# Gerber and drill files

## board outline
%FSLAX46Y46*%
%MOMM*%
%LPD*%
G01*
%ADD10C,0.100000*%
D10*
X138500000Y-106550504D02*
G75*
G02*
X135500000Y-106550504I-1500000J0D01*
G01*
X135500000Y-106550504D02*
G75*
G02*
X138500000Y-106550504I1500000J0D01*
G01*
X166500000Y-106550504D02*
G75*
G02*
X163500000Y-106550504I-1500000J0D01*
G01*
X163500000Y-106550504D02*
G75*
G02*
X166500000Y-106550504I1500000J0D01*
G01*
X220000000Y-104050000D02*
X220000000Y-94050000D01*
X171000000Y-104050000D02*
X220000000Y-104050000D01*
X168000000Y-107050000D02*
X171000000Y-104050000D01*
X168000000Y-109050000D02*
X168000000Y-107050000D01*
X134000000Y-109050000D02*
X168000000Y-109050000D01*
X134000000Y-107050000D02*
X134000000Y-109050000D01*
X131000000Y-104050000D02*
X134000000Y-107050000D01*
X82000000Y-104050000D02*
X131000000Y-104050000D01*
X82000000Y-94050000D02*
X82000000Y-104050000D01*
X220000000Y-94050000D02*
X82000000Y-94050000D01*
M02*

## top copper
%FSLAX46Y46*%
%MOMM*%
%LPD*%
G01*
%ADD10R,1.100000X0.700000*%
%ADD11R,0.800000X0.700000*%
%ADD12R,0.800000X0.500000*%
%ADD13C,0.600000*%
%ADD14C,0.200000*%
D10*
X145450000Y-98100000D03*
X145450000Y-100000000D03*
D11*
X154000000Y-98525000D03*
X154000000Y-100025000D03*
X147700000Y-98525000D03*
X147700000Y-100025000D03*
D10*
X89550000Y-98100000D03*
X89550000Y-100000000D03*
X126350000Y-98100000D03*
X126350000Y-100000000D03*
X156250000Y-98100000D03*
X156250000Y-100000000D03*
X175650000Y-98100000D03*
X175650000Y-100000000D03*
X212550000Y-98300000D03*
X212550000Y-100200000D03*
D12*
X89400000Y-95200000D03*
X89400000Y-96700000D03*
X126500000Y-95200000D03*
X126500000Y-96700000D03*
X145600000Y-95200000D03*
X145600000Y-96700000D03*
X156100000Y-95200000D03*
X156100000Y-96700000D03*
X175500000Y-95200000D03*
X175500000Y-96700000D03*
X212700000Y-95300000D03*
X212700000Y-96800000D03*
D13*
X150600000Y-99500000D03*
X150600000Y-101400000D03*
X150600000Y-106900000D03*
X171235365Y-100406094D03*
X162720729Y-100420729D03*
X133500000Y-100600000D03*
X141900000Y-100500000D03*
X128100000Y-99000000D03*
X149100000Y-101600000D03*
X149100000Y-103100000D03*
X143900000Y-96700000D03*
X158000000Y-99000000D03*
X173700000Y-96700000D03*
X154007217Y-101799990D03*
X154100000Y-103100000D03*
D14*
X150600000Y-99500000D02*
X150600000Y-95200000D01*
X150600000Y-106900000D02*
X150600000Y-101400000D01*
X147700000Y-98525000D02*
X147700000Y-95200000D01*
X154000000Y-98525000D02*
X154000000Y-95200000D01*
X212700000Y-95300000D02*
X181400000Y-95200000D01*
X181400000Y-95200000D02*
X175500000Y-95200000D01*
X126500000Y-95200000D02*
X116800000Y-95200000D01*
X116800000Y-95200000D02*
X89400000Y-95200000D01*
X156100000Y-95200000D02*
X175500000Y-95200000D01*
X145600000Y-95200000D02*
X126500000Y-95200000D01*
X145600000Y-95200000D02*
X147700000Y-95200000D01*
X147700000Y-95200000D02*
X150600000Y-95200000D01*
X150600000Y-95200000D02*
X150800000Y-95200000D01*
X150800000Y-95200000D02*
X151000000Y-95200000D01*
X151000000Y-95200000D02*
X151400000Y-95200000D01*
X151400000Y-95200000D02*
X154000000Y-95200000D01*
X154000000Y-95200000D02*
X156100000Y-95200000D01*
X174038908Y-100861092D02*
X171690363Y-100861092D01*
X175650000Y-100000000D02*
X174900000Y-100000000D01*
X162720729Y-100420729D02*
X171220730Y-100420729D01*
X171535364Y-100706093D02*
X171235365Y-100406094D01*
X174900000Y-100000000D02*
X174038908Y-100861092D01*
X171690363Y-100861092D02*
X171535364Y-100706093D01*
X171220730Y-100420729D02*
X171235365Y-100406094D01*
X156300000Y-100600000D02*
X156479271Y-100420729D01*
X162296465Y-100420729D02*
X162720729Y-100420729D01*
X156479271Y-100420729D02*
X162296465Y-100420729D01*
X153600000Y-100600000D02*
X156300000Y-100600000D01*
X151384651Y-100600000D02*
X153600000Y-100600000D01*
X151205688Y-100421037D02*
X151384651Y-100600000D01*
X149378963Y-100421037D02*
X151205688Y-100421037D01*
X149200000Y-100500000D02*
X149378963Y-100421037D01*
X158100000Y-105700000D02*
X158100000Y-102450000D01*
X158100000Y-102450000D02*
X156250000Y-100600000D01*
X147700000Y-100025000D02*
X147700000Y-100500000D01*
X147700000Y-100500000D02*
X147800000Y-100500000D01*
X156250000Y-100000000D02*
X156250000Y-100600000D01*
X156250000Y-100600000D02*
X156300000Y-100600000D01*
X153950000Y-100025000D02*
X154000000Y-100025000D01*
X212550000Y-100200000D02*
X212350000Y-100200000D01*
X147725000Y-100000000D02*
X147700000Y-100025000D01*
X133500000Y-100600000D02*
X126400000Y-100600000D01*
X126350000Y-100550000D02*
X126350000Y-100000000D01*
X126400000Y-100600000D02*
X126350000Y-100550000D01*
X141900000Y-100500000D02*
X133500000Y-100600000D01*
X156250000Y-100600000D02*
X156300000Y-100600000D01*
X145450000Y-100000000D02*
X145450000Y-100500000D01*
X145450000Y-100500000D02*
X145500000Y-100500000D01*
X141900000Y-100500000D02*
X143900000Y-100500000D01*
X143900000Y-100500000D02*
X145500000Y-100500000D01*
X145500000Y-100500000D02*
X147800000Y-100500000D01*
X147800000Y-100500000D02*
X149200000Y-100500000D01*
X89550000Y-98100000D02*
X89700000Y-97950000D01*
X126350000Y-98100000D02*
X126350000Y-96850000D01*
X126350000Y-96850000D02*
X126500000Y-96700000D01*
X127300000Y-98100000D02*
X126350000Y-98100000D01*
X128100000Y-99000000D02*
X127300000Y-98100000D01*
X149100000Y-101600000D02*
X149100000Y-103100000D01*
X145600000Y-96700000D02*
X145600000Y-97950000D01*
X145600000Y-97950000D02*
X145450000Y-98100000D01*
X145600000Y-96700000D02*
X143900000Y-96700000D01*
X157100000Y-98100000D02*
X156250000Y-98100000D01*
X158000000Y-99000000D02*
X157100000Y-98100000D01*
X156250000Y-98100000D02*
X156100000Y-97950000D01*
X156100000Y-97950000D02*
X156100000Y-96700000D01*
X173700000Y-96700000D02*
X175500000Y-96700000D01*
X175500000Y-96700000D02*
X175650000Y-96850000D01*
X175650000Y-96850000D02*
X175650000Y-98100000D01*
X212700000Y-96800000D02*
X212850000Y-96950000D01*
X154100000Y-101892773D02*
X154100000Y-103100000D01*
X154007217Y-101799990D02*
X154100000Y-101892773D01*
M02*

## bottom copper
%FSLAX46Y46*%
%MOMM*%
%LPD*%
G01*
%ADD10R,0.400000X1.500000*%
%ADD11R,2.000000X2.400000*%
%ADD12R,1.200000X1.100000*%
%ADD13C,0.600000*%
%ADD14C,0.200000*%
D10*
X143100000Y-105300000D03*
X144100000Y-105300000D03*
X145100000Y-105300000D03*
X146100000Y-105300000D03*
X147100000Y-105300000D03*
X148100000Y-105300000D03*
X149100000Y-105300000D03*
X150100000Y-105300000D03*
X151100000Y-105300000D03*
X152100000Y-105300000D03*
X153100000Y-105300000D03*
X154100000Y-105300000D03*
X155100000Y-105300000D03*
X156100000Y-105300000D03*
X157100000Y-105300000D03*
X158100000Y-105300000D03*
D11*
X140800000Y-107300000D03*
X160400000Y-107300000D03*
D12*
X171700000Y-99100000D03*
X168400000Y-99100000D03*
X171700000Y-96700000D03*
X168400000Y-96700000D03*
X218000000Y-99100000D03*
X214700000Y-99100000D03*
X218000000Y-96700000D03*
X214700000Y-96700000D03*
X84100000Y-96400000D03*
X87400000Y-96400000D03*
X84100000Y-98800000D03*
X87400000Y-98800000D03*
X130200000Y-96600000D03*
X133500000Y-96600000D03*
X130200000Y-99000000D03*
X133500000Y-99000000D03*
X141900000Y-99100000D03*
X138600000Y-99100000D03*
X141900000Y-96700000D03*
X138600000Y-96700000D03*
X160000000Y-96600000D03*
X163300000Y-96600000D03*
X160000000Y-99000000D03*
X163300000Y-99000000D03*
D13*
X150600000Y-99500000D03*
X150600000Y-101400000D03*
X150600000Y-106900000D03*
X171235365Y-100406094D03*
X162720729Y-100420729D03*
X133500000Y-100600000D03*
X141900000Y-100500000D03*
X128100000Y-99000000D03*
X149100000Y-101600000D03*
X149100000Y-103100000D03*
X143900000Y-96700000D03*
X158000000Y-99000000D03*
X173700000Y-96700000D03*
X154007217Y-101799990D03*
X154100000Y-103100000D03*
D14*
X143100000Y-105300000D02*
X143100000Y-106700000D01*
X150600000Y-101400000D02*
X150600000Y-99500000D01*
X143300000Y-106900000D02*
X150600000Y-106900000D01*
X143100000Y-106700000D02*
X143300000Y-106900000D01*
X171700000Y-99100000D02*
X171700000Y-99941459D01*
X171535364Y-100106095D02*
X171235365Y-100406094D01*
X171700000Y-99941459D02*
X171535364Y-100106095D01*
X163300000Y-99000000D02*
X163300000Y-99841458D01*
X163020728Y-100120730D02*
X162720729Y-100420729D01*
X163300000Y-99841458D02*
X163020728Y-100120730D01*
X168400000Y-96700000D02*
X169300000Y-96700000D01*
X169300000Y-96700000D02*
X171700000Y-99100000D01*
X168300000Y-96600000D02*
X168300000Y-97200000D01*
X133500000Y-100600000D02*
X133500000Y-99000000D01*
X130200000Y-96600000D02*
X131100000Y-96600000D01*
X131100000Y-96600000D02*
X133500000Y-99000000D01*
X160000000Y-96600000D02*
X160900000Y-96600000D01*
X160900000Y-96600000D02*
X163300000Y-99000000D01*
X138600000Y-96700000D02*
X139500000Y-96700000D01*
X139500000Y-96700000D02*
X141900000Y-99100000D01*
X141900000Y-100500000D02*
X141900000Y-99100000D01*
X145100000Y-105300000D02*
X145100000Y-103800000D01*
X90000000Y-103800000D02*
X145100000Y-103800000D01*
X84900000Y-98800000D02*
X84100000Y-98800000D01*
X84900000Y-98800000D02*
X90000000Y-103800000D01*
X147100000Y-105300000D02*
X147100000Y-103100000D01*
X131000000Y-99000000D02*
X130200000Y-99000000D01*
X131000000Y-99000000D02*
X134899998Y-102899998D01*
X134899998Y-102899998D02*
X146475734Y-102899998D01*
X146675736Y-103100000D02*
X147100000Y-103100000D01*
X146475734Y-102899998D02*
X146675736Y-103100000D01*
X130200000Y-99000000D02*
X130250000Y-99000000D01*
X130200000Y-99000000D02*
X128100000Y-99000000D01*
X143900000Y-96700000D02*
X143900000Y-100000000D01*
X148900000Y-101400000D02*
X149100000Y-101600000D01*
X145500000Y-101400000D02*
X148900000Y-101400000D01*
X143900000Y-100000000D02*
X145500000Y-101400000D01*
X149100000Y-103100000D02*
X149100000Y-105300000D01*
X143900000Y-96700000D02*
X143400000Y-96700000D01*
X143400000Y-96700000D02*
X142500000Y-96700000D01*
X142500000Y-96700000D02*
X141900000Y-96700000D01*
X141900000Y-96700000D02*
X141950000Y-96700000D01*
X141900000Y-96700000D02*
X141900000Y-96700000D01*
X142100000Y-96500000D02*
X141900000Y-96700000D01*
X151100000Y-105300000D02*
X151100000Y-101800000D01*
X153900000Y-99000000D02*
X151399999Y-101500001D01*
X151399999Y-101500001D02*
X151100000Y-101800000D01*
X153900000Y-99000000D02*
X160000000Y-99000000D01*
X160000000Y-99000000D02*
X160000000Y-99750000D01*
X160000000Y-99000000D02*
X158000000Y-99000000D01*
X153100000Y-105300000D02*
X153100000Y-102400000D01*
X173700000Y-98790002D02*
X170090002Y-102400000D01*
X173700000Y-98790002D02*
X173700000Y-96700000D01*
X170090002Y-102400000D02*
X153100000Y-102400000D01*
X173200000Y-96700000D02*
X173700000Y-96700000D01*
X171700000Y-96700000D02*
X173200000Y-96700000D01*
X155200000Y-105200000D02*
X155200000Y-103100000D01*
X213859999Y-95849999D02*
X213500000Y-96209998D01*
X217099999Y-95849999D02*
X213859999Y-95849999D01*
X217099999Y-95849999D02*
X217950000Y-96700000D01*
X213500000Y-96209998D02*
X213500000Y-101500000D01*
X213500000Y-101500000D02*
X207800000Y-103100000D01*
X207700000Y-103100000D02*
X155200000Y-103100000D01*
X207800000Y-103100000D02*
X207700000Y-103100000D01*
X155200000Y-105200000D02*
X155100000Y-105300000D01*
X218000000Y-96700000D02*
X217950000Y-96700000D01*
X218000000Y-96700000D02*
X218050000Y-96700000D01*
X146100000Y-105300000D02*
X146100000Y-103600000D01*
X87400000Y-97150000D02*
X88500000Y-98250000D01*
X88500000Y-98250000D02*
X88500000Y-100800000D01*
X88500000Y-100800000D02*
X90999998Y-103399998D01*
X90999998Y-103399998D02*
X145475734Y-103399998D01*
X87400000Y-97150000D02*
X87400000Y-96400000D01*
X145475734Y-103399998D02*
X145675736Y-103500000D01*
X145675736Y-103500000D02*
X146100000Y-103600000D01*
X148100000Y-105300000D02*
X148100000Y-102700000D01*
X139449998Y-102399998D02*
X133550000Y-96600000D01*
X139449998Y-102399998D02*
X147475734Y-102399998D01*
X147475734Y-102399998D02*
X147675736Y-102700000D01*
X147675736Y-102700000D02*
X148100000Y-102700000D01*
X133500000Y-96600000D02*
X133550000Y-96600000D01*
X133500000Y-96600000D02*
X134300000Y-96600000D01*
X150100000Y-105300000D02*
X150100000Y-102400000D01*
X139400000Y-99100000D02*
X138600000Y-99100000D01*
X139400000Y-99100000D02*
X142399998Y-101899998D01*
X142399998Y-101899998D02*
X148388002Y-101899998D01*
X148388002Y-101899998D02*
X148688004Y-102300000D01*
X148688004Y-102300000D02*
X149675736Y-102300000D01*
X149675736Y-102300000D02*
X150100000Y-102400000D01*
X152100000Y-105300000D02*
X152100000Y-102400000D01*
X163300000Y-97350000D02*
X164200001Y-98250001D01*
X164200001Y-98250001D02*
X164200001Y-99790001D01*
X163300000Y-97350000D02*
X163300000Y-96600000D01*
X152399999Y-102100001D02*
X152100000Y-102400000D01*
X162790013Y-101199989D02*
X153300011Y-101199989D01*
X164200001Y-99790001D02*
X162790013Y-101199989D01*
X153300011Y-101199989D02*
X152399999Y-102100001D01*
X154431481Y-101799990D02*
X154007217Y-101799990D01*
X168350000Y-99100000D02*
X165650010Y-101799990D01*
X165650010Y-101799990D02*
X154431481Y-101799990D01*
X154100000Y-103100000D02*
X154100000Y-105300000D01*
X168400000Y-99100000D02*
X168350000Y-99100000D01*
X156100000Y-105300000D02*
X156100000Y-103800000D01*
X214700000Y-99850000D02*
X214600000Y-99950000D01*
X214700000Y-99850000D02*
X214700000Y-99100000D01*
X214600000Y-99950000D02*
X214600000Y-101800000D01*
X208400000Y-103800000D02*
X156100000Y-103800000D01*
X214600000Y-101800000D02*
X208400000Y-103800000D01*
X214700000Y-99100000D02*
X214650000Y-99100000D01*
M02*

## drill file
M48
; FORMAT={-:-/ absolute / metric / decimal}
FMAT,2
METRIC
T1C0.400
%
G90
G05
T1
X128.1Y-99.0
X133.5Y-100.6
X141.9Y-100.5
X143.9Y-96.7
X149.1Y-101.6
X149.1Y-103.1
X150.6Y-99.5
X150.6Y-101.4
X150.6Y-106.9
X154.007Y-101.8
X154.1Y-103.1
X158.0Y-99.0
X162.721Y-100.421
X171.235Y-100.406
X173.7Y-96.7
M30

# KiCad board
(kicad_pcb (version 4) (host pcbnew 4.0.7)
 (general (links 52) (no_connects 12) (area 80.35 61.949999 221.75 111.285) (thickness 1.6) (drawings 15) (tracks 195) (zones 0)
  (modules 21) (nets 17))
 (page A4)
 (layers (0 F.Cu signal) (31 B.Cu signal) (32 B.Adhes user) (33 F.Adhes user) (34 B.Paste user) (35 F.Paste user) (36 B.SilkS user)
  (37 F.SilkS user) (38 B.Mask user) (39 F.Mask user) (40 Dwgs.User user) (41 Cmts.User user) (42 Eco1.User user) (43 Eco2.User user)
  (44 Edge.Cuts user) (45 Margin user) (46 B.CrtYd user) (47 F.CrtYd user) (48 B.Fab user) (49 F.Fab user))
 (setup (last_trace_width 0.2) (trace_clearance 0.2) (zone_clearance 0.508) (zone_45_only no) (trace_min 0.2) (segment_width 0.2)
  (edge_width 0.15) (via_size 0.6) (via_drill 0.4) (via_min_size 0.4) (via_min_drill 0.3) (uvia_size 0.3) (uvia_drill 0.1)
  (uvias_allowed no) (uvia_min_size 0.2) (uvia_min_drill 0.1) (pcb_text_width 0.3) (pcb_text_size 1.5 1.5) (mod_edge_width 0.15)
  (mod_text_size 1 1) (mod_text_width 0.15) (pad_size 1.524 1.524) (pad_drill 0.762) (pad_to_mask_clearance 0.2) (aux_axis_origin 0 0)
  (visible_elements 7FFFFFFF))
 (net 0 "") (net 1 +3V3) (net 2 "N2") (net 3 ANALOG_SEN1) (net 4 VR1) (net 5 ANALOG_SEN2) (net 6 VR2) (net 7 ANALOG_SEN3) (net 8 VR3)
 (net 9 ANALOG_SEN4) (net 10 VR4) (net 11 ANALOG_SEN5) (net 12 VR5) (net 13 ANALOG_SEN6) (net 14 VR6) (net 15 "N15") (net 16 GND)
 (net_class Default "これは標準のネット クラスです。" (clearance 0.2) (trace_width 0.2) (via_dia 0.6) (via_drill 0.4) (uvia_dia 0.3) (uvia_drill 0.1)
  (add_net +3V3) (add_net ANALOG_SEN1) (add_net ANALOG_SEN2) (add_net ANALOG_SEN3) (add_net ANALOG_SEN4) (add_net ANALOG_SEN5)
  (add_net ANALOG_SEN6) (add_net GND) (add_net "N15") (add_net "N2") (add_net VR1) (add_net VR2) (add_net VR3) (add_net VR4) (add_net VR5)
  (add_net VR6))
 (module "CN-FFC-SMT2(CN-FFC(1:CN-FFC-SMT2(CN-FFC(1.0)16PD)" (layer F.Cu) (at 140.1 110.3)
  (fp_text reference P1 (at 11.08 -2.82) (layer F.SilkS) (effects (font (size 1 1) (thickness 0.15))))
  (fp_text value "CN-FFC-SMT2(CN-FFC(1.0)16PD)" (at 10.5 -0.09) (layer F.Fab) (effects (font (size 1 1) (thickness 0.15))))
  (pad 1 smd rect (at 3 -5) (size 0.4 1.5) (layers B.Cu B.Paste B.Mask) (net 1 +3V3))
  (pad 2 smd rect (at 4 -5) (size 0.4 1.5) (layers B.Cu B.Paste B.Mask) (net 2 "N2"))
  (pad 3 smd rect (at 5 -5) (size 0.4 1.5) (layers B.Cu B.Paste B.Mask) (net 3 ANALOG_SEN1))
  (pad 4 smd rect (at 6 -5) (size 0.4 1.5) (layers B.Cu B.Paste B.Mask) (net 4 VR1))
  (pad 5 smd rect (at 7 -5) (size 0.4 1.5) (layers B.Cu B.Paste B.Mask) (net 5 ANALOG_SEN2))
  (pad 6 smd rect (at 8 -5) (size 0.4 1.5) (layers B.Cu B.Paste B.Mask) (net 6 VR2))
  (pad 7 smd rect (at 9 -5) (size 0.4 1.5) (layers B.Cu B.Paste B.Mask) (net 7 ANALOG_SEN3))
  (pad 8 smd rect (at 10 -5) (size 0.4 1.5) (layers B.Cu B.Paste B.Mask) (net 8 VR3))
  (pad 9 smd rect (at 11 -5) (size 0.4 1.5) (layers B.Cu B.Paste B.Mask) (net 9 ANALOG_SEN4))
  (pad 10 smd rect (at 12 -5) (size 0.4 1.5) (layers B.Cu B.Paste B.Mask) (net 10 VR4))
  (pad 11 smd rect (at 13 -5) (size 0.4 1.5) (layers B.Cu B.Paste B.Mask) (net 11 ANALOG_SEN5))
  (pad 12 smd rect (at 14 -5) (size 0.4 1.5) (layers B.Cu B.Paste B.Mask) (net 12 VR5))
  (pad 13 smd rect (at 15 -5) (size 0.4 1.5) (layers B.Cu B.Paste B.Mask) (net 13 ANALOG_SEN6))
  (pad 14 smd rect (at 16 -5) (size 0.4 1.5) (layers B.Cu B.Paste B.Mask) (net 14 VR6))
  (pad 15 smd rect (at 17 -5) (size 0.4 1.5) (layers B.Cu B.Paste B.Mask) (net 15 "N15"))
  (pad 16 smd rect (at 18 -5) (size 0.4 1.5) (layers B.Cu B.Paste B.Mask) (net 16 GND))
  (pad "" smd rect (at 0.7 -3) (size 2 2.4) (layers B.Cu B.Paste B.Mask))
  (pad "" smd rect (at 20.3 -3) (size 2 2.4) (layers B.Cu B.Paste B.Mask)))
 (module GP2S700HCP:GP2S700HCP (layer F.Cu) (at 175 93.1 180)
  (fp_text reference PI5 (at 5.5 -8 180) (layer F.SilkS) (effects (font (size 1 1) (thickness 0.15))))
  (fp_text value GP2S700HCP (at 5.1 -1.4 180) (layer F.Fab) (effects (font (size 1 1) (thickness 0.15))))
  (pad 1 smd rect (at 3.3 -6 180) (size 1.2 1.1) (layers B.Cu B.Paste B.Mask) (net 16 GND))
  (pad 4 smd rect (at 6.6 -6 180) (size 1.2 1.1) (layers B.Cu B.Paste B.Mask) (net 12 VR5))
  (pad 2 smd rect (at 3.3 -3.6 180) (size 1.2 1.1) (layers B.Cu B.Paste B.Mask) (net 11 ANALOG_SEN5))
  (pad 3 smd rect (at 6.6 -3.6 180) (size 1.2 1.1) (layers B.Cu B.Paste B.Mask) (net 16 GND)))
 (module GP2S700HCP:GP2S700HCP (layer F.Cu) (at 221.3 93.1 180)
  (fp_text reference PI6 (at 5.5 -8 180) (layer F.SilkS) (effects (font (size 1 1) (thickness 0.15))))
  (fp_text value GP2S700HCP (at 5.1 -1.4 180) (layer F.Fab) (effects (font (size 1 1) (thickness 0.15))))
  (pad 1 smd rect (at 3.3 -6 180) (size 1.2 1.1) (layers B.Cu B.Paste B.Mask) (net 16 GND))
  (pad 4 smd rect (at 6.6 -6 180) (size 1.2 1.1) (layers B.Cu B.Paste B.Mask) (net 14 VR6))
  (pad 2 smd rect (at 3.3 -3.6 180) (size 1.2 1.1) (layers B.Cu B.Paste B.Mask) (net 13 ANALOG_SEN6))
  (pad 3 smd rect (at 6.6 -3.6 180) (size 1.2 1.1) (layers B.Cu B.Paste B.Mask) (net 16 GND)))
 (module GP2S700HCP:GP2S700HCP (layer F.Cu) (at 80.8 102.4)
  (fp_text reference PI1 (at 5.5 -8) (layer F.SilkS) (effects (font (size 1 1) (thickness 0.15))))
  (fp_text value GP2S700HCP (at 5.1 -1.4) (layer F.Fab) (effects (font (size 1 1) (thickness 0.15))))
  (pad 1 smd rect (at 3.3 -6) (size 1.2 1.1) (layers B.Cu B.Paste B.Mask) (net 16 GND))
  (pad 4 smd rect (at 6.6 -6) (size 1.2 1.1) (layers B.Cu B.Paste B.Mask) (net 4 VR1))
  (pad 2 smd rect (at 3.3 -3.6) (size 1.2 1.1) (layers B.Cu B.Paste B.Mask) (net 3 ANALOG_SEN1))
  (pad 3 smd rect (at 6.6 -3.6) (size 1.2 1.1) (layers B.Cu B.Paste B.Mask) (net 16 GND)))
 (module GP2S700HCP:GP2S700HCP (layer F.Cu) (at 126.9 102.6)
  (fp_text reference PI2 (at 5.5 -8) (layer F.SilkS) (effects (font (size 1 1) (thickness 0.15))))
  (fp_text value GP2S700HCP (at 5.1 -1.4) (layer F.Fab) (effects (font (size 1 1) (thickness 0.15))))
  (pad 1 smd rect (at 3.3 -6) (size 1.2 1.1) (layers B.Cu B.Paste B.Mask) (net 16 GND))
  (pad 4 smd rect (at 6.6 -6) (size 1.2 1.1) (layers B.Cu B.Paste B.Mask) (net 6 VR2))
  (pad 2 smd rect (at 3.3 -3.6) (size 1.2 1.1) (layers B.Cu B.Paste B.Mask) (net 5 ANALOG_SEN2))
  (pad 3 smd rect (at 6.6 -3.6) (size 1.2 1.1) (layers B.Cu B.Paste B.Mask) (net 16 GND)))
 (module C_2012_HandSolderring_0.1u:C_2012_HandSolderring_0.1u (layer F.Cu) (at 143.5 96.7 270)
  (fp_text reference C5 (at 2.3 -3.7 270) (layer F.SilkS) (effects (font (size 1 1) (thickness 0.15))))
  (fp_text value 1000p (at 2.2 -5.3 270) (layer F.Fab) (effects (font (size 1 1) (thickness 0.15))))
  (pad 1 smd rect (at 1.4 -1.95 270) (size 0.7 1.1) (layers F.Cu F.Paste F.Mask) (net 7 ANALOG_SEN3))
  (pad 2 smd rect (at 3.3 -1.95 270) (size 0.7 1.1) (layers F.Cu F.Paste F.Mask) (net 16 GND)))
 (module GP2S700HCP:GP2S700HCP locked (layer F.Cu) (at 145.2 93.1 180)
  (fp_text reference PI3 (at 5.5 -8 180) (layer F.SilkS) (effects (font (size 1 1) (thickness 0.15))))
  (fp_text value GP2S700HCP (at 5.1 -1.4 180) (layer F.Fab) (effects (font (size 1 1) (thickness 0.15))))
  (pad 1 smd rect (at 3.3 -6 180) (size 1.2 1.1) (layers B.Cu B.Paste B.Mask) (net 16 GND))
  (pad 4 smd rect (at 6.6 -6 180) (size 1.2 1.1) (layers B.Cu B.Paste B.Mask) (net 8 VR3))
  (pad 2 smd rect (at 3.3 -3.6 180) (size 1.2 1.1) (layers B.Cu B.Paste B.Mask) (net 7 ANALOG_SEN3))
  (pad 3 smd rect (at 6.6 -3.6 180) (size 1.2 1.1) (layers B.Cu B.Paste B.Mask) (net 16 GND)))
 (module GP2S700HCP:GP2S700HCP (layer F.Cu) (at 156.7 102.6)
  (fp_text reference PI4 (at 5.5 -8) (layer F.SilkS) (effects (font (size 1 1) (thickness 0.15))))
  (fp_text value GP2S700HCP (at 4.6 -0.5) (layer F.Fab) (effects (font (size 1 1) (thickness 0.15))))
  (pad 1 smd rect (at 3.3 -6) (size 1.2 1.1) (layers B.Cu B.Paste B.Mask) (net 16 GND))
  (pad 4 smd rect (at 6.6 -6) (size 1.2 1.1) (layers B.Cu B.Paste B.Mask) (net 10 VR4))
  (pad 2 smd rect (at 3.3 -3.6) (size 1.2 1.1) (layers B.Cu B.Paste B.Mask) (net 9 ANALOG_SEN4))
  (pad 3 smd rect (at 6.6 -3.6) (size 1.2 1.1) (layers B.Cu B.Paste B.Mask) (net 16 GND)))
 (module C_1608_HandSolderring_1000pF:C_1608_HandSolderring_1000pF (layer F.Cu) (at 153.1 97.9 270)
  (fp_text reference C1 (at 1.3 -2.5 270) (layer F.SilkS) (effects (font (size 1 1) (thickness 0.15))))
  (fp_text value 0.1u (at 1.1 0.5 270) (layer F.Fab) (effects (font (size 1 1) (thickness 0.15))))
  (pad 1 smd rect (at 0.625 -0.9 270) (size 0.7 0.8) (layers F.Cu F.Paste F.Mask) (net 1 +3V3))
  (pad 2 smd rect (at 2.125 -0.9 270) (size 0.7 0.8) (layers F.Cu F.Paste F.Mask) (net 16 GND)))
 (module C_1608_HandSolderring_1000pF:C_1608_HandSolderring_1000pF (layer F.Cu) (at 146.8 97.9 270)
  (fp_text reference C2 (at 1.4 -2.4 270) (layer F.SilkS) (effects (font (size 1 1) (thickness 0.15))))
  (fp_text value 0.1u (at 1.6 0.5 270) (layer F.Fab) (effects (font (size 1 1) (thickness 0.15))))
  (pad 1 smd rect (at 0.625 -0.9 270) (size 0.7 0.8) (layers F.Cu F.Paste F.Mask) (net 1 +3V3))
  (pad 2 smd rect (at 2.125 -0.9 270) (size 0.7 0.8) (layers F.Cu F.Paste F.Mask) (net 16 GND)))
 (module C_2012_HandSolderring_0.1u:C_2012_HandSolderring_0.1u (layer F.Cu) (at 87.6 96.7 270)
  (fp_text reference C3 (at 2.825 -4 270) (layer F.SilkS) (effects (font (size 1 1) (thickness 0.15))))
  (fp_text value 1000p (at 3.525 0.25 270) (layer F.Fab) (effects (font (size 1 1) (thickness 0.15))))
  (pad 1 smd rect (at 1.4 -1.95 270) (size 0.7 1.1) (layers F.Cu F.Paste F.Mask) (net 3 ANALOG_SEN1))
  (pad 2 smd rect (at 3.3 -1.95 270) (size 0.7 1.1) (layers F.Cu F.Paste F.Mask) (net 16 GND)))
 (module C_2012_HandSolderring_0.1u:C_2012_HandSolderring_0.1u (layer F.Cu) (at 124.4 96.7 270)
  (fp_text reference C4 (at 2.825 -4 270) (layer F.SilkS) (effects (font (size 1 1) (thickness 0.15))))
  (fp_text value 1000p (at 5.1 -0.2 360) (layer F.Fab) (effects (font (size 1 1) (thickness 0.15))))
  (pad 1 smd rect (at 1.4 -1.95 270) (size 0.7 1.1) (layers F.Cu F.Paste F.Mask) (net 5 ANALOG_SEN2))
  (pad 2 smd rect (at 3.3 -1.95 270) (size 0.7 1.1) (layers F.Cu F.Paste F.Mask) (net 16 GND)))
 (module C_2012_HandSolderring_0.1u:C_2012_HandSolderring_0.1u (layer F.Cu) (at 154.3 96.7 270)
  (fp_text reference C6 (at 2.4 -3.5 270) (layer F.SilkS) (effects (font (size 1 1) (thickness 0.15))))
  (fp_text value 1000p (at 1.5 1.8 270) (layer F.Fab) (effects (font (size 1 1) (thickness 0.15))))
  (pad 1 smd rect (at 1.4 -1.95 270) (size 0.7 1.1) (layers F.Cu F.Paste F.Mask) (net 9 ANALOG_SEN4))
  (pad 2 smd rect (at 3.3 -1.95 270) (size 0.7 1.1) (layers F.Cu F.Paste F.Mask) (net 16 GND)))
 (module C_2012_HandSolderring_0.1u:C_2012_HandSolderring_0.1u (layer F.Cu) (at 173.7 96.7 270)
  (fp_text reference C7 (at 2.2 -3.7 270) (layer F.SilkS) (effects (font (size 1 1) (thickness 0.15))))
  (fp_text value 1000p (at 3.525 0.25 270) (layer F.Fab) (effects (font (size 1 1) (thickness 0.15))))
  (pad 1 smd rect (at 1.4 -1.95 270) (size 0.7 1.1) (layers F.Cu F.Paste F.Mask) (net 11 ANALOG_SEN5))
  (pad 2 smd rect (at 3.3 -1.95 270) (size 0.7 1.1) (layers F.Cu F.Paste F.Mask) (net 16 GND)))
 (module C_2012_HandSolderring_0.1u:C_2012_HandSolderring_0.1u (layer F.Cu) (at 210.6 96.9 270)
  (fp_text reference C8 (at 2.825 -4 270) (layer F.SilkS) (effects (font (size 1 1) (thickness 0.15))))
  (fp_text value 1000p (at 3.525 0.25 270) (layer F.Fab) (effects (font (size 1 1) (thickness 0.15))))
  (pad 1 smd rect (at 1.4 -1.95 270) (size 0.7 1.1) (layers F.Cu F.Paste F.Mask) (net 13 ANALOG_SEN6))
  (pad 2 smd rect (at 3.3 -1.95 270) (size 0.7 1.1) (layers F.Cu F.Paste F.Mask) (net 16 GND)))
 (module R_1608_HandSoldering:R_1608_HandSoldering (layer F.Cu) (at 87.8 93.8 270)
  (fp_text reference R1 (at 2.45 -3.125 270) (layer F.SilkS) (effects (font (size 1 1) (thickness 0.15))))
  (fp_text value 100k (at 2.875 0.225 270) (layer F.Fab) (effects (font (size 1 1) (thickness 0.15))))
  (pad 1 smd rect (at 1.4 -1.6 270) (size 0.5 0.8) (layers F.Cu F.Paste F.Mask) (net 1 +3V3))
  (pad 2 smd rect (at 2.9 -1.6 270) (size 0.5 0.8) (layers F.Cu F.Paste F.Mask) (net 3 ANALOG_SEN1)))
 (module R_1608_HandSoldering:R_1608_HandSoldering (layer F.Cu) (at 124.9 93.8 270)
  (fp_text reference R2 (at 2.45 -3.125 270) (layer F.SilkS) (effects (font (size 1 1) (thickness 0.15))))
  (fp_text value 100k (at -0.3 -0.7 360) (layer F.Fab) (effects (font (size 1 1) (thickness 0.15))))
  (pad 1 smd rect (at 1.4 -1.6 270) (size 0.5 0.8) (layers F.Cu F.Paste F.Mask) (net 1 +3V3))
  (pad 2 smd rect (at 2.9 -1.6 270) (size 0.5 0.8) (layers F.Cu F.Paste F.Mask) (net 5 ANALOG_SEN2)))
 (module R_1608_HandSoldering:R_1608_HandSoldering (layer F.Cu) (at 144 93.8 270)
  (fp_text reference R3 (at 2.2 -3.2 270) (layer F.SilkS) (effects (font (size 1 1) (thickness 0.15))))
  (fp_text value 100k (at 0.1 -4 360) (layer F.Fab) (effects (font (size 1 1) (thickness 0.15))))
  (pad 1 smd rect (at 1.4 -1.6 270) (size 0.5 0.8) (layers F.Cu F.Paste F.Mask) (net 1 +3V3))
  (pad 2 smd rect (at 2.9 -1.6 270) (size 0.5 0.8) (layers F.Cu F.Paste F.Mask) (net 7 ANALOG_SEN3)))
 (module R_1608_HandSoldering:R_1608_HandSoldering (layer F.Cu) (at 154.5 93.8 270)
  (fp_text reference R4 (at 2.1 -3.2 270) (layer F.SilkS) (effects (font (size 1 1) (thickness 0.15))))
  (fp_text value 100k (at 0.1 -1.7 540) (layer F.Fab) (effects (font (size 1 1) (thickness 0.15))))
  (pad 1 smd rect (at 1.4 -1.6 270) (size 0.5 0.8) (layers F.Cu F.Paste F.Mask) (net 1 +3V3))
  (pad 2 smd rect (at 2.9 -1.6 270) (size 0.5 0.8) (layers F.Cu F.Paste F.Mask) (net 9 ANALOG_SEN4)))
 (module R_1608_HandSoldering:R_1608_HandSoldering (layer F.Cu) (at 173.9 93.8 270)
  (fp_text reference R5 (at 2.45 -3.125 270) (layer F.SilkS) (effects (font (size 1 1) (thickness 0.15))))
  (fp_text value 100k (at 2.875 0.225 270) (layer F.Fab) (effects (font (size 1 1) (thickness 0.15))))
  (pad 1 smd rect (at 1.4 -1.6 270) (size 0.5 0.8) (layers F.Cu F.Paste F.Mask) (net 1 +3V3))
  (pad 2 smd rect (at 2.9 -1.6 270) (size 0.5 0.8) (layers F.Cu F.Paste F.Mask) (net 11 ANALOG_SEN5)))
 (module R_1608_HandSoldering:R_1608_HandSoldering (layer F.Cu) (at 211.1 93.9 270)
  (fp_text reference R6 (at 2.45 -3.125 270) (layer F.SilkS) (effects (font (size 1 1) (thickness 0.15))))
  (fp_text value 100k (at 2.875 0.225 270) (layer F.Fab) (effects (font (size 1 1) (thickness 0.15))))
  (pad 1 smd rect (at 1.4 -1.6 270) (size 0.5 0.8) (layers F.Cu F.Paste F.Mask) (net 1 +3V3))
  (pad 2 smd rect (at 2.9 -1.6 270) (size 0.5 0.8) (layers F.Cu F.Paste F.Mask) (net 13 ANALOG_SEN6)))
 (gr_circle (center 137 106.550504) (end 137 105.050504) (layer Edge.Cuts) (width 0.1))
 (gr_circle (center 165 106.550504) (end 165 105.050504) (layer Edge.Cuts) (width 0.1))
 (gr_line (start 220 104.05) (end 220 94.05) (layer Edge.Cuts) (width 0.1))
 (gr_line (start 171 104.05) (end 220 104.05) (layer Edge.Cuts) (width 0.1))
 (gr_line (start 168 107.05) (end 171 104.05) (layer Edge.Cuts) (width 0.1))
 (gr_line (start 168 109.05) (end 168 107.05) (layer Edge.Cuts) (width 0.1))
 (gr_line (start 134 109.05) (end 168 109.05) (layer Edge.Cuts) (width 0.1))
 (gr_line (start 134 107.05) (end 134 109.05) (layer Edge.Cuts) (width 0.1))
 (gr_line (start 131 104.05) (end 134 107.05) (layer Edge.Cuts) (width 0.1))
 (gr_line (start 82 104.05) (end 131 104.05) (layer Edge.Cuts) (width 0.1))
 (gr_line (start 82 94.05) (end 82 104.05) (layer Edge.Cuts) (width 0.1))
 (gr_line (start 220 94.05) (end 82 94.05) (layer Edge.Cuts) (width 0.1))
 (segment (start 143.1 105.3) (end 143.1 106.7) (width 0.2) (layer B.Cu) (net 1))
 (segment (start 150.6 99.5) (end 150.6 95.2) (width 0.2) (layer F.Cu) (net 1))
 (via (at 150.6 99.5) (size 0.6) (drill 0.4) (layers F.Cu B.Cu) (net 1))
 (segment (start 150.6 101.4) (end 150.6 99.5) (width 0.2) (layer B.Cu) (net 1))
 (via (at 150.6 101.4) (size 0.6) (drill 0.4) (layers F.Cu B.Cu) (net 1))
 (segment (start 150.6 106.9) (end 150.6 101.4) (width 0.2) (layer F.Cu) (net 1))
 (via (at 150.6 106.9) (size 0.6) (drill 0.4) (layers F.Cu B.Cu) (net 1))
 (segment (start 143.3 106.9) (end 150.6 106.9) (width 0.2) (layer B.Cu) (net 1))
 (segment (start 143.1 106.7) (end 143.3 106.9) (width 0.2) (layer B.Cu) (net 1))
 (segment (start 147.7 98.525) (end 147.7 95.2) (width 0.2) (layer F.Cu) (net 1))
 (segment (start 154 98.525) (end 154 95.2) (width 0.2) (layer F.Cu) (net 1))
 (segment (start 212.7 95.3) (end 181.4 95.2) (width 0.2) (layer F.Cu) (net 1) (status 10))
 (segment (start 181.4 95.2) (end 175.5 95.2) (width 0.2) (layer F.Cu) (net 1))
 (segment (start 126.5 95.2) (end 116.8 95.2) (width 0.2) (layer F.Cu) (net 1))
 (segment (start 116.8 95.2) (end 89.4 95.2) (width 0.2) (layer F.Cu) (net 1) (status 20))
 (segment (start 156.1 95.2) (end 175.5 95.2) (width 0.2) (layer F.Cu) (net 1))
 (segment (start 145.6 95.2) (end 126.5 95.2) (width 0.2) (layer F.Cu) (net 1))
 (segment (start 145.6 95.2) (end 147.7 95.2) (width 0.2) (layer F.Cu) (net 1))
 (segment (start 147.7 95.2) (end 150.6 95.2) (width 0.2) (layer F.Cu) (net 1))
 (segment (start 150.6 95.2) (end 150.8 95.2) (width 0.2) (layer F.Cu) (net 1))
 (segment (start 150.8 95.2) (end 151 95.2) (width 0.2) (layer F.Cu) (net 1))
 (segment (start 151 95.2) (end 151.4 95.2) (width 0.2) (layer F.Cu) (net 1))
 (segment (start 151.4 95.2) (end 154 95.2) (width 0.2) (layer F.Cu) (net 1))
 (segment (start 154 95.2) (end 156.1 95.2) (width 0.2) (layer F.Cu) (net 1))
 (segment (start 174.038908 100.861092) (end 171.690363 100.861092) (width 0.2) (layer F.Cu) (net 16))
 (segment (start 175.65 100) (end 174.9 100) (width 0.2) (layer F.Cu) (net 16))
 (segment (start 171.7 99.1) (end 171.7 99.941459) (width 0.2) (layer B.Cu) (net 16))
 (segment (start 162.720729 100.420729) (end 171.22073 100.420729) (width 0.2) (layer F.Cu) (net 16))
 (segment (start 171.535364 100.706093) (end 171.235365 100.406094) (width 0.2) (layer F.Cu) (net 16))
 (segment (start 174.9 100) (end 174.038908 100.861092) (width 0.2) (layer F.Cu) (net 16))
 (segment (start 171.535364 100.106095) (end 171.235365 100.406094) (width 0.2) (layer B.Cu) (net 16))
 (segment (start 171.690363 100.861092) (end 171.535364 100.706093) (width 0.2) (layer F.Cu) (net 16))
 (segment (start 171.22073 100.420729) (end 171.235365 100.406094) (width 0.2) (layer F.Cu) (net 16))
 (via (at 171.235365 100.406094) (size 0.6) (drill 0.4) (layers F.Cu B.Cu) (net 16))
 (segment (start 171.7 99.941459) (end 171.535364 100.106095) (width 0.2) (layer B.Cu) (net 16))
 (segment (start 156.3 100.6) (end 156.479271 100.420729) (width 0.2) (layer F.Cu) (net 16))
 (segment (start 163.3 99) (end 163.3 99.841458) (width 0.2) (layer B.Cu) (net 16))
 (segment (start 163.020728 100.12073) (end 162.720729 100.420729) (width 0.2) (layer B.Cu) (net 16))
 (via (at 162.720729 100.420729) (size 0.6) (drill 0.4) (layers F.Cu B.Cu) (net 16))
 (segment (start 162.296465 100.420729) (end 162.720729 100.420729) (width 0.2) (layer F.Cu) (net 16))
 (segment (start 156.479271 100.420729) (end 162.296465 100.420729) (width 0.2) (layer F.Cu) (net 16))
 (segment (start 163.3 99.841458) (end 163.020728 100.12073) (width 0.2) (layer B.Cu) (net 16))
 (segment (start 153.6 100.6) (end 156.3 100.6) (width 0.2) (layer F.Cu) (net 16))
 (segment (start 151.384651 100.6) (end 153.6 100.6) (width 0.2) (layer F.Cu) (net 16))
 (segment (start 151.205688 100.421037) (end 151.384651 100.6) (width 0.2) (layer F.Cu) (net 16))
 (segment (start 149.378963 100.421037) (end 151.205688 100.421037) (width 0.2) (layer F.Cu) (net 16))
 (segment (start 149.2 100.5) (end 149.378963 100.421037) (width 0.2) (layer F.Cu) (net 16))
 (segment (start 158.1 105.7) (end 158.1 102.45) (width 0.2) (layer F.Cu) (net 16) (status 10))
 (segment (start 158.1 102.45) (end 156.25 100.6) (width 0.2) (layer F.Cu) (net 16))
 (segment (start 147.7 100.025) (end 147.7 100.5) (width 0.2) (layer F.Cu) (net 16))
 (segment (start 147.7 100.5) (end 147.8 100.5) (width 0.2) (layer F.Cu) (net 16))
 (segment (start 156.25 100) (end 156.25 100.6) (width 0.2) (layer F.Cu) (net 16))
 (segment (start 156.25 100.6) (end 156.3 100.6) (width 0.2) (layer F.Cu) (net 16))
 (segment (start 168.4 96.7) (end 169.3 96.7) (width 0.2) (layer B.Cu) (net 16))
 (segment (start 169.3 96.7) (end 171.7 99.1) (width 0.2) (layer B.Cu) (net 16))
 (segment (start 153.95 100.025) (end 154 100.025) (width 0.2) (layer F.Cu) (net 16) (status 30))
 (segment (start 212.55 100.2) (end 212.35 100.2) (width 0.2) (layer F.Cu) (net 16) (status 30))
 (segment (start 168.3 96.6) (end 168.3 97.2) (width 0.2) (layer B.Cu) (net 16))
 (segment (start 147.725 100) (end 147.7 100.025) (width 0.2) (layer F.Cu) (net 16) (status 30))
 (segment (start 133.5 100.6) (end 126.4 100.6) (width 0.2) (layer F.Cu) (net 16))
 (segment (start 126.35 100.55) (end 126.35 100) (width 0.2) (layer F.Cu) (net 16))
 (segment (start 126.4 100.6) (end 126.35 100.55) (width 0.2) (layer F.Cu) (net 16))
 (segment (start 141.9 100.5) (end 133.5 100.6) (width 0.2) (layer F.Cu) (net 16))
 (segment (start 133.5 100.6) (end 133.5 99) (width 0.2) (layer B.Cu) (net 16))
 (via (at 133.5 100.6) (size 0.6) (drill 0.4) (layers F.Cu B.Cu) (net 16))
 (segment (start 130.2 96.6) (end 131.1 96.6) (width 0.2) (layer B.Cu) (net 16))
 (segment (start 131.1 96.6) (end 133.5 99) (width 0.2) (layer B.Cu) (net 16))
 (segment (start 156.25 100.6) (end 156.3 100.6) (width 0.2) (layer F.Cu) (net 16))
 (segment (start 145.45 100) (end 145.45 100.5) (width 0.2) (layer F.Cu) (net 16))
 (segment (start 145.45 100.5) (end 145.5 100.5) (width 0.2) (layer F.Cu) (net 16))
 (segment (start 160 96.6) (end 160.9 96.6) (width 0.2) (layer B.Cu) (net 16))
 (segment (start 160.9 96.6) (end 163.3 99) (width 0.2) (layer B.Cu) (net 16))
 (segment (start 138.6 96.7) (end 139.5 96.7) (width 0.2) (layer B.Cu) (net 16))
 (segment (start 139.5 96.7) (end 141.9 99.1) (width 0.2) (layer B.Cu) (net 16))
 (segment (start 141.9 100.5) (end 143.9 100.5) (width 0.2) (layer F.Cu) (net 16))
 (segment (start 143.9 100.5) (end 145.5 100.5) (width 0.2) (layer F.Cu) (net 16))
 (segment (start 145.5 100.5) (end 147.8 100.5) (width 0.2) (layer F.Cu) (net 16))
 (segment (start 147.8 100.5) (end 149.2 100.5) (width 0.2) (layer F.Cu) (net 16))
 (segment (start 141.9 100.5) (end 141.9 99.1) (width 0.2) (layer B.Cu) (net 16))
 (via (at 141.9 100.5) (size 0.6) (drill 0.4) (layers F.Cu B.Cu) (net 16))
 (segment (start 145.1 105.3) (end 145.1 103.8) (width 0.2) (layer B.Cu) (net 3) (status 10))
 (segment (start 90 103.8) (end 145.1 103.8) (width 0.2) (layer B.Cu) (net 3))
 (segment (start 84.9 98.8) (end 84.1 98.8) (width 0.2) (layer B.Cu) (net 3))
 (segment (start 84.9 98.8) (end 90 103.8) (width 0.2) (layer B.Cu) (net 3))
 (segment (start 89.55 98.1) (end 89.7 97.95) (width 0.2) (layer F.Cu) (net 3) (status 30))
 (segment (start 147.1 105.3) (end 147.1 103.1) (width 0.2) (layer B.Cu) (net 5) (status 10))
 (segment (start 131 99) (end 130.2 99) (width 0.2) (layer B.Cu) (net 5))
 (segment (start 131 99) (end 134.899998 102.899998) (width 0.2) (layer B.Cu) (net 5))
 (segment (start 134.899998 102.899998) (end 146.475734 102.899998) (width 0.2) (layer B.Cu) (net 5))
 (segment (start 146.675736 103.1) (end 147.1 103.1) (width 0.2) (layer B.Cu) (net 5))
 (segment (start 146.475734 102.899998) (end 146.675736 103.1) (width 0.2) (layer B.Cu) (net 5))
 (segment (start 130.2 99) (end 130.25 99) (width 0.2) (layer B.Cu) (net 5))
 (segment (start 130.2 99) (end 128.1 99) (width 0.2) (layer B.Cu) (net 5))
 (via (at 128.1 99) (size 0.6) (drill 0.4) (layers F.Cu B.Cu) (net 5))
 (segment (start 126.35 98.1) (end 126.35 96.85) (width 0.2) (layer F.Cu) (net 5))
 (segment (start 126.35 96.85) (end 126.5 96.7) (width 0.2) (layer F.Cu) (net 5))
 (segment (start 127.3 98.1) (end 126.35 98.1) (width 0.2) (layer F.Cu) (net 5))
 (segment (start 128.1 99) (end 127.3 98.1) (width 0.2) (layer F.Cu) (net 5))
 (via (at 149.1 101.6) (size 0.6) (drill 0.4) (layers F.Cu B.Cu) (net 7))
 (segment (start 143.9 96.7) (end 143.9 100) (width 0.2) (layer B.Cu) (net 7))
 (segment (start 148.9 101.4) (end 149.1 101.6) (width 0.2) (layer B.Cu) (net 7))
 (segment (start 145.5 101.4) (end 148.9 101.4) (width 0.2) (layer B.Cu) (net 7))
 (segment (start 143.9 100) (end 145.5 101.4) (width 0.2) (layer B.Cu) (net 7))
 (segment (start 149.1 103.1) (end 149.1 105.3) (width 0.2) (layer B.Cu) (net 7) (status 20))
 (via (at 149.1 103.1) (size 0.6) (drill 0.4) (layers F.Cu B.Cu) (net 7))
 (segment (start 149.1 101.6) (end 149.1 103.1) (width 0.2) (layer F.Cu) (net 7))
 (segment (start 143.9 96.7) (end 143.4 96.7) (width 0.2) (layer B.Cu) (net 7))
 (segment (start 143.4 96.7) (end 142.5 96.7) (width 0.2) (layer B.Cu) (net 7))
 (segment (start 142.5 96.7) (end 141.9 96.7) (width 0.2) (layer B.Cu) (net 7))
 (segment (start 141.9 96.7) (end 141.95 96.7) (width 0.2) (layer B.Cu) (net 7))
 (segment (start 141.9 96.7) (end 141.9 96.7) (width 0.2) (layer B.Cu) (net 7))
 (segment (start 145.6 96.7) (end 145.6 97.95) (width 0.2) (layer F.Cu) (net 7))
 (segment (start 145.6 97.95) (end 145.45 98.1) (width 0.2) (layer F.Cu) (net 7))
 (segment (start 145.6 96.7) (end 143.9 96.7) (width 0.2) (layer F.Cu) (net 7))
 (via (at 143.9 96.7) (size 0.6) (drill 0.4) (layers F.Cu B.Cu) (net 7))
 (segment (start 142.1 96.5) (end 141.9 96.7) (width 0.2) (layer B.Cu) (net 7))
 (segment (start 151.1 105.3) (end 151.1 101.8) (width 0.2) (layer B.Cu) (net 9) (status 10))
 (segment (start 153.9 99) (end 151.399999 101.500001) (width 0.2) (layer B.Cu) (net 9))
 (segment (start 151.399999 101.500001) (end 151.1 101.8) (width 0.2) (layer B.Cu) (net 9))
 (segment (start 153.9 99) (end 160 99) (width 0.2) (layer B.Cu) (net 9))
 (segment (start 160 99) (end 160 99.75) (width 0.2) (layer B.Cu) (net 9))
 (segment (start 160 99) (end 158 99) (width 0.2) (layer B.Cu) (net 9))
 (segment (start 157.1 98.1) (end 156.25 98.1) (width 0.2) (layer F.Cu) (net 9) (status 20))
 (segment (start 158 99) (end 157.1 98.1) (width 0.2) (layer F.Cu) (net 9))
 (via (at 158 99) (size 0.6) (drill 0.4) (layers F.Cu B.Cu) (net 9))
 (segment (start 156.25 98.1) (end 156.1 97.95) (width 0.2) (layer F.Cu) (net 9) (status 30))
 (segment (start 156.1 97.95) (end 156.1 96.7) (width 0.2) (layer F.Cu) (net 9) (status 20))
 (segment (start 153.1 105.3) (end 153.1 102.4) (width 0.2) (layer B.Cu) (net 11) (status 10))
 (segment (start 173.7 98.790002) (end 170.090002 102.4) (width 0.2) (layer B.Cu) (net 11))
 (segment (start 173.7 98.790002) (end 173.7 96.7) (width 0.2) (layer B.Cu) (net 11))
 (segment (start 170.090002 102.4) (end 153.1 102.4) (width 0.2) (layer B.Cu) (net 11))
 (segment (start 173.2 96.7) (end 173.7 96.7) (width 0.2) (layer B.Cu) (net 11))
 (segment (start 171.7 96.7) (end 173.2 96.7) (width 0.2) (layer B.Cu) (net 11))
 (segment (start 173.7 96.7) (end 175.5 96.7) (width 0.2) (layer F.Cu) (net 11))
 (via (at 173.7 96.7) (size 0.6) (drill 0.4) (layers F.Cu B.Cu) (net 11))
 (segment (start 175.5 96.7) (end 175.65 96.85) (width 0.2) (layer F.Cu) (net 11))
 (segment (start 175.65 96.85) (end 175.65 98.1) (width 0.2) (layer F.Cu) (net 11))
 (segment (start 155.2 105.2) (end 155.2 103.1) (width 0.2) (layer B.Cu) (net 13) (status 10))
 (segment (start 213.859999 95.849999) (end 213.5 96.209998) (width 0.2) (layer B.Cu) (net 13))
 (segment (start 217.099999 95.849999) (end 213.859999 95.849999) (width 0.2) (layer B.Cu) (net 13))
 (segment (start 217.099999 95.849999) (end 217.95 96.7) (width 0.2) (layer B.Cu) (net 13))
 (segment (start 213.5 96.209998) (end 213.5 101.5) (width 0.2) (layer B.Cu) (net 13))
 (segment (start 213.5 101.5) (end 207.8 103.1) (width 0.2) (layer B.Cu) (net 13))
 (segment (start 207.7 103.1) (end 155.2 103.1) (width 0.2) (layer B.Cu) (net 13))
 (segment (start 207.8 103.1) (end 207.7 103.1) (width 0.2) (layer B.Cu) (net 13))
 (segment (start 155.2 105.2) (end 155.1 105.3) (width 0.2) (layer B.Cu) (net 13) (status 30))
 (segment (start 218 96.7) (end 217.95 96.7) (width 0.2) (layer B.Cu) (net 13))
 (segment (start 218 96.7) (end 218.05 96.7) (width 0.2) (layer B.Cu) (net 13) (status 30))
 (segment (start 212.7 96.8) (end 212.85 96.95) (width 0.2) (layer F.Cu) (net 13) (status 30))
 (segment (start 146.1 105.3) (end 146.1 103.6) (width 0.2) (layer B.Cu) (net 4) (status 10))
 (segment (start 87.4 97.15) (end 88.5 98.25) (width 0.2) (layer B.Cu) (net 4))
 (segment (start 88.5 98.25) (end 88.5 100.8) (width 0.2) (layer B.Cu) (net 4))
 (segment (start 88.5 100.8) (end 90.999998 103.399998) (width 0.2) (layer B.Cu) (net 4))
 (segment (start 90.999998 103.399998) (end 145.475734 103.399998) (width 0.2) (layer B.Cu) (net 4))
 (segment (start 87.4 97.15) (end 87.4 96.4) (width 0.2) (layer B.Cu) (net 4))
 (segment (start 145.475734 103.399998) (end 145.675736 103.5) (width 0.2) (layer B.Cu) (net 4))
 (segment (start 145.675736 103.5) (end 146.1 103.6) (width 0.2) (layer B.Cu) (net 4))
 (segment (start 148.1 105.3) (end 148.1 102.7) (width 0.2) (layer B.Cu) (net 6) (status 10))
 (segment (start 139.449998 102.399998) (end 133.55 96.6) (width 0.2) (layer B.Cu) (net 6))
 (segment (start 139.449998 102.399998) (end 147.475734 102.399998) (width 0.2) (layer B.Cu) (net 6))
 (segment (start 147.475734 102.399998) (end 147.675736 102.7) (width 0.2) (layer B.Cu) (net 6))
 (segment (start 147.675736 102.7) (end 148.1 102.7) (width 0.2) (layer B.Cu) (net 6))
 (segment (start 133.5 96.6) (end 133.55 96.6) (width 0.2) (layer B.Cu) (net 6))
 (segment (start 133.5 96.6) (end 134.3 96.6) (width 0.2) (layer B.Cu) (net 6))
 (segment (start 150.1 105.3) (end 150.1 102.4) (width 0.2) (layer B.Cu) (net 8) (status 10))
 (segment (start 139.4 99.1) (end 138.6 99.1) (width 0.2) (layer B.Cu) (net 8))
 (segment (start 139.4 99.1) (end 142.399998 101.899998) (width 0.2) (layer B.Cu) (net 8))
 (segment (start 142.399998 101.899998) (end 148.388002 101.899998) (width 0.2) (layer B.Cu) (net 8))
 (segment (start 148.388002 101.899998) (end 148.688004 102.3) (width 0.2) (layer B.Cu) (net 8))
 (segment (start 148.688004 102.3) (end 149.675736 102.3) (width 0.2) (layer B.Cu) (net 8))
 (segment (start 149.675736 102.3) (end 150.1 102.4) (width 0.2) (layer B.Cu) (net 8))
 (segment (start 152.1 105.3) (end 152.1 102.4) (width 0.2) (layer B.Cu) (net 10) (status 10))
 (segment (start 163.3 97.35) (end 164.200001 98.250001) (width 0.2) (layer B.Cu) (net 10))
 (segment (start 164.200001 98.250001) (end 164.200001 99.790001) (width 0.2) (layer B.Cu) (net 10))
 (segment (start 163.3 97.35) (end 163.3 96.6) (width 0.2) (layer B.Cu) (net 10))
 (segment (start 152.399999 102.100001) (end 152.1 102.4) (width 0.2) (layer B.Cu) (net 10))
 (segment (start 162.790013 101.199989) (end 153.300011 101.199989) (width 0.2) (layer B.Cu) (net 10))
 (segment (start 164.200001 99.790001) (end 162.790013 101.199989) (width 0.2) (layer B.Cu) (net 10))
 (segment (start 153.300011 101.199989) (end 152.399999 102.100001) (width 0.2) (layer B.Cu) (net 10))
 (via (at 154.007217 101.79999) (size 0.6) (drill 0.4) (layers F.Cu B.Cu) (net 12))
 (segment (start 154.431481 101.79999) (end 154.007217 101.79999) (width 0.2) (layer B.Cu) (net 12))
 (segment (start 168.35 99.1) (end 165.65001 101.79999) (width 0.2) (layer B.Cu) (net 12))
 (segment (start 165.65001 101.79999) (end 154.431481 101.79999) (width 0.2) (layer B.Cu) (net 12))
 (segment (start 154.1 103.1) (end 154.1 105.3) (width 0.2) (layer B.Cu) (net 12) (status 20))
 (via (at 154.1 103.1) (size 0.6) (drill 0.4) (layers F.Cu B.Cu) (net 12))
 (segment (start 154.1 101.892773) (end 154.1 103.1) (width 0.2) (layer F.Cu) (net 12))
 (segment (start 154.007217 101.79999) (end 154.1 101.892773) (width 0.2) (layer F.Cu) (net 12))
 (segment (start 168.4 99.1) (end 168.35 99.1) (width 0.2) (layer B.Cu) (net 12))
 (segment (start 156.1 105.3) (end 156.1 103.8) (width 0.2) (layer B.Cu) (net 14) (status 10))
 (segment (start 214.7 99.85) (end 214.6 99.95) (width 0.2) (layer B.Cu) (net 14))
 (segment (start 214.7 99.85) (end 214.7 99.1) (width 0.2) (layer B.Cu) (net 14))
 (segment (start 214.6 99.95) (end 214.6 101.8) (width 0.2) (layer B.Cu) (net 14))
 (segment (start 208.4 103.8) (end 156.1 103.8) (width 0.2) (layer B.Cu) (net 14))
 (segment (start 214.6 101.8) (end 208.4 103.8) (width 0.2) (layer B.Cu) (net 14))
 (segment (start 214.7 99.1) (end 214.65 99.1) (width 0.2) (layer B.Cu) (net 14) (status 30)))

